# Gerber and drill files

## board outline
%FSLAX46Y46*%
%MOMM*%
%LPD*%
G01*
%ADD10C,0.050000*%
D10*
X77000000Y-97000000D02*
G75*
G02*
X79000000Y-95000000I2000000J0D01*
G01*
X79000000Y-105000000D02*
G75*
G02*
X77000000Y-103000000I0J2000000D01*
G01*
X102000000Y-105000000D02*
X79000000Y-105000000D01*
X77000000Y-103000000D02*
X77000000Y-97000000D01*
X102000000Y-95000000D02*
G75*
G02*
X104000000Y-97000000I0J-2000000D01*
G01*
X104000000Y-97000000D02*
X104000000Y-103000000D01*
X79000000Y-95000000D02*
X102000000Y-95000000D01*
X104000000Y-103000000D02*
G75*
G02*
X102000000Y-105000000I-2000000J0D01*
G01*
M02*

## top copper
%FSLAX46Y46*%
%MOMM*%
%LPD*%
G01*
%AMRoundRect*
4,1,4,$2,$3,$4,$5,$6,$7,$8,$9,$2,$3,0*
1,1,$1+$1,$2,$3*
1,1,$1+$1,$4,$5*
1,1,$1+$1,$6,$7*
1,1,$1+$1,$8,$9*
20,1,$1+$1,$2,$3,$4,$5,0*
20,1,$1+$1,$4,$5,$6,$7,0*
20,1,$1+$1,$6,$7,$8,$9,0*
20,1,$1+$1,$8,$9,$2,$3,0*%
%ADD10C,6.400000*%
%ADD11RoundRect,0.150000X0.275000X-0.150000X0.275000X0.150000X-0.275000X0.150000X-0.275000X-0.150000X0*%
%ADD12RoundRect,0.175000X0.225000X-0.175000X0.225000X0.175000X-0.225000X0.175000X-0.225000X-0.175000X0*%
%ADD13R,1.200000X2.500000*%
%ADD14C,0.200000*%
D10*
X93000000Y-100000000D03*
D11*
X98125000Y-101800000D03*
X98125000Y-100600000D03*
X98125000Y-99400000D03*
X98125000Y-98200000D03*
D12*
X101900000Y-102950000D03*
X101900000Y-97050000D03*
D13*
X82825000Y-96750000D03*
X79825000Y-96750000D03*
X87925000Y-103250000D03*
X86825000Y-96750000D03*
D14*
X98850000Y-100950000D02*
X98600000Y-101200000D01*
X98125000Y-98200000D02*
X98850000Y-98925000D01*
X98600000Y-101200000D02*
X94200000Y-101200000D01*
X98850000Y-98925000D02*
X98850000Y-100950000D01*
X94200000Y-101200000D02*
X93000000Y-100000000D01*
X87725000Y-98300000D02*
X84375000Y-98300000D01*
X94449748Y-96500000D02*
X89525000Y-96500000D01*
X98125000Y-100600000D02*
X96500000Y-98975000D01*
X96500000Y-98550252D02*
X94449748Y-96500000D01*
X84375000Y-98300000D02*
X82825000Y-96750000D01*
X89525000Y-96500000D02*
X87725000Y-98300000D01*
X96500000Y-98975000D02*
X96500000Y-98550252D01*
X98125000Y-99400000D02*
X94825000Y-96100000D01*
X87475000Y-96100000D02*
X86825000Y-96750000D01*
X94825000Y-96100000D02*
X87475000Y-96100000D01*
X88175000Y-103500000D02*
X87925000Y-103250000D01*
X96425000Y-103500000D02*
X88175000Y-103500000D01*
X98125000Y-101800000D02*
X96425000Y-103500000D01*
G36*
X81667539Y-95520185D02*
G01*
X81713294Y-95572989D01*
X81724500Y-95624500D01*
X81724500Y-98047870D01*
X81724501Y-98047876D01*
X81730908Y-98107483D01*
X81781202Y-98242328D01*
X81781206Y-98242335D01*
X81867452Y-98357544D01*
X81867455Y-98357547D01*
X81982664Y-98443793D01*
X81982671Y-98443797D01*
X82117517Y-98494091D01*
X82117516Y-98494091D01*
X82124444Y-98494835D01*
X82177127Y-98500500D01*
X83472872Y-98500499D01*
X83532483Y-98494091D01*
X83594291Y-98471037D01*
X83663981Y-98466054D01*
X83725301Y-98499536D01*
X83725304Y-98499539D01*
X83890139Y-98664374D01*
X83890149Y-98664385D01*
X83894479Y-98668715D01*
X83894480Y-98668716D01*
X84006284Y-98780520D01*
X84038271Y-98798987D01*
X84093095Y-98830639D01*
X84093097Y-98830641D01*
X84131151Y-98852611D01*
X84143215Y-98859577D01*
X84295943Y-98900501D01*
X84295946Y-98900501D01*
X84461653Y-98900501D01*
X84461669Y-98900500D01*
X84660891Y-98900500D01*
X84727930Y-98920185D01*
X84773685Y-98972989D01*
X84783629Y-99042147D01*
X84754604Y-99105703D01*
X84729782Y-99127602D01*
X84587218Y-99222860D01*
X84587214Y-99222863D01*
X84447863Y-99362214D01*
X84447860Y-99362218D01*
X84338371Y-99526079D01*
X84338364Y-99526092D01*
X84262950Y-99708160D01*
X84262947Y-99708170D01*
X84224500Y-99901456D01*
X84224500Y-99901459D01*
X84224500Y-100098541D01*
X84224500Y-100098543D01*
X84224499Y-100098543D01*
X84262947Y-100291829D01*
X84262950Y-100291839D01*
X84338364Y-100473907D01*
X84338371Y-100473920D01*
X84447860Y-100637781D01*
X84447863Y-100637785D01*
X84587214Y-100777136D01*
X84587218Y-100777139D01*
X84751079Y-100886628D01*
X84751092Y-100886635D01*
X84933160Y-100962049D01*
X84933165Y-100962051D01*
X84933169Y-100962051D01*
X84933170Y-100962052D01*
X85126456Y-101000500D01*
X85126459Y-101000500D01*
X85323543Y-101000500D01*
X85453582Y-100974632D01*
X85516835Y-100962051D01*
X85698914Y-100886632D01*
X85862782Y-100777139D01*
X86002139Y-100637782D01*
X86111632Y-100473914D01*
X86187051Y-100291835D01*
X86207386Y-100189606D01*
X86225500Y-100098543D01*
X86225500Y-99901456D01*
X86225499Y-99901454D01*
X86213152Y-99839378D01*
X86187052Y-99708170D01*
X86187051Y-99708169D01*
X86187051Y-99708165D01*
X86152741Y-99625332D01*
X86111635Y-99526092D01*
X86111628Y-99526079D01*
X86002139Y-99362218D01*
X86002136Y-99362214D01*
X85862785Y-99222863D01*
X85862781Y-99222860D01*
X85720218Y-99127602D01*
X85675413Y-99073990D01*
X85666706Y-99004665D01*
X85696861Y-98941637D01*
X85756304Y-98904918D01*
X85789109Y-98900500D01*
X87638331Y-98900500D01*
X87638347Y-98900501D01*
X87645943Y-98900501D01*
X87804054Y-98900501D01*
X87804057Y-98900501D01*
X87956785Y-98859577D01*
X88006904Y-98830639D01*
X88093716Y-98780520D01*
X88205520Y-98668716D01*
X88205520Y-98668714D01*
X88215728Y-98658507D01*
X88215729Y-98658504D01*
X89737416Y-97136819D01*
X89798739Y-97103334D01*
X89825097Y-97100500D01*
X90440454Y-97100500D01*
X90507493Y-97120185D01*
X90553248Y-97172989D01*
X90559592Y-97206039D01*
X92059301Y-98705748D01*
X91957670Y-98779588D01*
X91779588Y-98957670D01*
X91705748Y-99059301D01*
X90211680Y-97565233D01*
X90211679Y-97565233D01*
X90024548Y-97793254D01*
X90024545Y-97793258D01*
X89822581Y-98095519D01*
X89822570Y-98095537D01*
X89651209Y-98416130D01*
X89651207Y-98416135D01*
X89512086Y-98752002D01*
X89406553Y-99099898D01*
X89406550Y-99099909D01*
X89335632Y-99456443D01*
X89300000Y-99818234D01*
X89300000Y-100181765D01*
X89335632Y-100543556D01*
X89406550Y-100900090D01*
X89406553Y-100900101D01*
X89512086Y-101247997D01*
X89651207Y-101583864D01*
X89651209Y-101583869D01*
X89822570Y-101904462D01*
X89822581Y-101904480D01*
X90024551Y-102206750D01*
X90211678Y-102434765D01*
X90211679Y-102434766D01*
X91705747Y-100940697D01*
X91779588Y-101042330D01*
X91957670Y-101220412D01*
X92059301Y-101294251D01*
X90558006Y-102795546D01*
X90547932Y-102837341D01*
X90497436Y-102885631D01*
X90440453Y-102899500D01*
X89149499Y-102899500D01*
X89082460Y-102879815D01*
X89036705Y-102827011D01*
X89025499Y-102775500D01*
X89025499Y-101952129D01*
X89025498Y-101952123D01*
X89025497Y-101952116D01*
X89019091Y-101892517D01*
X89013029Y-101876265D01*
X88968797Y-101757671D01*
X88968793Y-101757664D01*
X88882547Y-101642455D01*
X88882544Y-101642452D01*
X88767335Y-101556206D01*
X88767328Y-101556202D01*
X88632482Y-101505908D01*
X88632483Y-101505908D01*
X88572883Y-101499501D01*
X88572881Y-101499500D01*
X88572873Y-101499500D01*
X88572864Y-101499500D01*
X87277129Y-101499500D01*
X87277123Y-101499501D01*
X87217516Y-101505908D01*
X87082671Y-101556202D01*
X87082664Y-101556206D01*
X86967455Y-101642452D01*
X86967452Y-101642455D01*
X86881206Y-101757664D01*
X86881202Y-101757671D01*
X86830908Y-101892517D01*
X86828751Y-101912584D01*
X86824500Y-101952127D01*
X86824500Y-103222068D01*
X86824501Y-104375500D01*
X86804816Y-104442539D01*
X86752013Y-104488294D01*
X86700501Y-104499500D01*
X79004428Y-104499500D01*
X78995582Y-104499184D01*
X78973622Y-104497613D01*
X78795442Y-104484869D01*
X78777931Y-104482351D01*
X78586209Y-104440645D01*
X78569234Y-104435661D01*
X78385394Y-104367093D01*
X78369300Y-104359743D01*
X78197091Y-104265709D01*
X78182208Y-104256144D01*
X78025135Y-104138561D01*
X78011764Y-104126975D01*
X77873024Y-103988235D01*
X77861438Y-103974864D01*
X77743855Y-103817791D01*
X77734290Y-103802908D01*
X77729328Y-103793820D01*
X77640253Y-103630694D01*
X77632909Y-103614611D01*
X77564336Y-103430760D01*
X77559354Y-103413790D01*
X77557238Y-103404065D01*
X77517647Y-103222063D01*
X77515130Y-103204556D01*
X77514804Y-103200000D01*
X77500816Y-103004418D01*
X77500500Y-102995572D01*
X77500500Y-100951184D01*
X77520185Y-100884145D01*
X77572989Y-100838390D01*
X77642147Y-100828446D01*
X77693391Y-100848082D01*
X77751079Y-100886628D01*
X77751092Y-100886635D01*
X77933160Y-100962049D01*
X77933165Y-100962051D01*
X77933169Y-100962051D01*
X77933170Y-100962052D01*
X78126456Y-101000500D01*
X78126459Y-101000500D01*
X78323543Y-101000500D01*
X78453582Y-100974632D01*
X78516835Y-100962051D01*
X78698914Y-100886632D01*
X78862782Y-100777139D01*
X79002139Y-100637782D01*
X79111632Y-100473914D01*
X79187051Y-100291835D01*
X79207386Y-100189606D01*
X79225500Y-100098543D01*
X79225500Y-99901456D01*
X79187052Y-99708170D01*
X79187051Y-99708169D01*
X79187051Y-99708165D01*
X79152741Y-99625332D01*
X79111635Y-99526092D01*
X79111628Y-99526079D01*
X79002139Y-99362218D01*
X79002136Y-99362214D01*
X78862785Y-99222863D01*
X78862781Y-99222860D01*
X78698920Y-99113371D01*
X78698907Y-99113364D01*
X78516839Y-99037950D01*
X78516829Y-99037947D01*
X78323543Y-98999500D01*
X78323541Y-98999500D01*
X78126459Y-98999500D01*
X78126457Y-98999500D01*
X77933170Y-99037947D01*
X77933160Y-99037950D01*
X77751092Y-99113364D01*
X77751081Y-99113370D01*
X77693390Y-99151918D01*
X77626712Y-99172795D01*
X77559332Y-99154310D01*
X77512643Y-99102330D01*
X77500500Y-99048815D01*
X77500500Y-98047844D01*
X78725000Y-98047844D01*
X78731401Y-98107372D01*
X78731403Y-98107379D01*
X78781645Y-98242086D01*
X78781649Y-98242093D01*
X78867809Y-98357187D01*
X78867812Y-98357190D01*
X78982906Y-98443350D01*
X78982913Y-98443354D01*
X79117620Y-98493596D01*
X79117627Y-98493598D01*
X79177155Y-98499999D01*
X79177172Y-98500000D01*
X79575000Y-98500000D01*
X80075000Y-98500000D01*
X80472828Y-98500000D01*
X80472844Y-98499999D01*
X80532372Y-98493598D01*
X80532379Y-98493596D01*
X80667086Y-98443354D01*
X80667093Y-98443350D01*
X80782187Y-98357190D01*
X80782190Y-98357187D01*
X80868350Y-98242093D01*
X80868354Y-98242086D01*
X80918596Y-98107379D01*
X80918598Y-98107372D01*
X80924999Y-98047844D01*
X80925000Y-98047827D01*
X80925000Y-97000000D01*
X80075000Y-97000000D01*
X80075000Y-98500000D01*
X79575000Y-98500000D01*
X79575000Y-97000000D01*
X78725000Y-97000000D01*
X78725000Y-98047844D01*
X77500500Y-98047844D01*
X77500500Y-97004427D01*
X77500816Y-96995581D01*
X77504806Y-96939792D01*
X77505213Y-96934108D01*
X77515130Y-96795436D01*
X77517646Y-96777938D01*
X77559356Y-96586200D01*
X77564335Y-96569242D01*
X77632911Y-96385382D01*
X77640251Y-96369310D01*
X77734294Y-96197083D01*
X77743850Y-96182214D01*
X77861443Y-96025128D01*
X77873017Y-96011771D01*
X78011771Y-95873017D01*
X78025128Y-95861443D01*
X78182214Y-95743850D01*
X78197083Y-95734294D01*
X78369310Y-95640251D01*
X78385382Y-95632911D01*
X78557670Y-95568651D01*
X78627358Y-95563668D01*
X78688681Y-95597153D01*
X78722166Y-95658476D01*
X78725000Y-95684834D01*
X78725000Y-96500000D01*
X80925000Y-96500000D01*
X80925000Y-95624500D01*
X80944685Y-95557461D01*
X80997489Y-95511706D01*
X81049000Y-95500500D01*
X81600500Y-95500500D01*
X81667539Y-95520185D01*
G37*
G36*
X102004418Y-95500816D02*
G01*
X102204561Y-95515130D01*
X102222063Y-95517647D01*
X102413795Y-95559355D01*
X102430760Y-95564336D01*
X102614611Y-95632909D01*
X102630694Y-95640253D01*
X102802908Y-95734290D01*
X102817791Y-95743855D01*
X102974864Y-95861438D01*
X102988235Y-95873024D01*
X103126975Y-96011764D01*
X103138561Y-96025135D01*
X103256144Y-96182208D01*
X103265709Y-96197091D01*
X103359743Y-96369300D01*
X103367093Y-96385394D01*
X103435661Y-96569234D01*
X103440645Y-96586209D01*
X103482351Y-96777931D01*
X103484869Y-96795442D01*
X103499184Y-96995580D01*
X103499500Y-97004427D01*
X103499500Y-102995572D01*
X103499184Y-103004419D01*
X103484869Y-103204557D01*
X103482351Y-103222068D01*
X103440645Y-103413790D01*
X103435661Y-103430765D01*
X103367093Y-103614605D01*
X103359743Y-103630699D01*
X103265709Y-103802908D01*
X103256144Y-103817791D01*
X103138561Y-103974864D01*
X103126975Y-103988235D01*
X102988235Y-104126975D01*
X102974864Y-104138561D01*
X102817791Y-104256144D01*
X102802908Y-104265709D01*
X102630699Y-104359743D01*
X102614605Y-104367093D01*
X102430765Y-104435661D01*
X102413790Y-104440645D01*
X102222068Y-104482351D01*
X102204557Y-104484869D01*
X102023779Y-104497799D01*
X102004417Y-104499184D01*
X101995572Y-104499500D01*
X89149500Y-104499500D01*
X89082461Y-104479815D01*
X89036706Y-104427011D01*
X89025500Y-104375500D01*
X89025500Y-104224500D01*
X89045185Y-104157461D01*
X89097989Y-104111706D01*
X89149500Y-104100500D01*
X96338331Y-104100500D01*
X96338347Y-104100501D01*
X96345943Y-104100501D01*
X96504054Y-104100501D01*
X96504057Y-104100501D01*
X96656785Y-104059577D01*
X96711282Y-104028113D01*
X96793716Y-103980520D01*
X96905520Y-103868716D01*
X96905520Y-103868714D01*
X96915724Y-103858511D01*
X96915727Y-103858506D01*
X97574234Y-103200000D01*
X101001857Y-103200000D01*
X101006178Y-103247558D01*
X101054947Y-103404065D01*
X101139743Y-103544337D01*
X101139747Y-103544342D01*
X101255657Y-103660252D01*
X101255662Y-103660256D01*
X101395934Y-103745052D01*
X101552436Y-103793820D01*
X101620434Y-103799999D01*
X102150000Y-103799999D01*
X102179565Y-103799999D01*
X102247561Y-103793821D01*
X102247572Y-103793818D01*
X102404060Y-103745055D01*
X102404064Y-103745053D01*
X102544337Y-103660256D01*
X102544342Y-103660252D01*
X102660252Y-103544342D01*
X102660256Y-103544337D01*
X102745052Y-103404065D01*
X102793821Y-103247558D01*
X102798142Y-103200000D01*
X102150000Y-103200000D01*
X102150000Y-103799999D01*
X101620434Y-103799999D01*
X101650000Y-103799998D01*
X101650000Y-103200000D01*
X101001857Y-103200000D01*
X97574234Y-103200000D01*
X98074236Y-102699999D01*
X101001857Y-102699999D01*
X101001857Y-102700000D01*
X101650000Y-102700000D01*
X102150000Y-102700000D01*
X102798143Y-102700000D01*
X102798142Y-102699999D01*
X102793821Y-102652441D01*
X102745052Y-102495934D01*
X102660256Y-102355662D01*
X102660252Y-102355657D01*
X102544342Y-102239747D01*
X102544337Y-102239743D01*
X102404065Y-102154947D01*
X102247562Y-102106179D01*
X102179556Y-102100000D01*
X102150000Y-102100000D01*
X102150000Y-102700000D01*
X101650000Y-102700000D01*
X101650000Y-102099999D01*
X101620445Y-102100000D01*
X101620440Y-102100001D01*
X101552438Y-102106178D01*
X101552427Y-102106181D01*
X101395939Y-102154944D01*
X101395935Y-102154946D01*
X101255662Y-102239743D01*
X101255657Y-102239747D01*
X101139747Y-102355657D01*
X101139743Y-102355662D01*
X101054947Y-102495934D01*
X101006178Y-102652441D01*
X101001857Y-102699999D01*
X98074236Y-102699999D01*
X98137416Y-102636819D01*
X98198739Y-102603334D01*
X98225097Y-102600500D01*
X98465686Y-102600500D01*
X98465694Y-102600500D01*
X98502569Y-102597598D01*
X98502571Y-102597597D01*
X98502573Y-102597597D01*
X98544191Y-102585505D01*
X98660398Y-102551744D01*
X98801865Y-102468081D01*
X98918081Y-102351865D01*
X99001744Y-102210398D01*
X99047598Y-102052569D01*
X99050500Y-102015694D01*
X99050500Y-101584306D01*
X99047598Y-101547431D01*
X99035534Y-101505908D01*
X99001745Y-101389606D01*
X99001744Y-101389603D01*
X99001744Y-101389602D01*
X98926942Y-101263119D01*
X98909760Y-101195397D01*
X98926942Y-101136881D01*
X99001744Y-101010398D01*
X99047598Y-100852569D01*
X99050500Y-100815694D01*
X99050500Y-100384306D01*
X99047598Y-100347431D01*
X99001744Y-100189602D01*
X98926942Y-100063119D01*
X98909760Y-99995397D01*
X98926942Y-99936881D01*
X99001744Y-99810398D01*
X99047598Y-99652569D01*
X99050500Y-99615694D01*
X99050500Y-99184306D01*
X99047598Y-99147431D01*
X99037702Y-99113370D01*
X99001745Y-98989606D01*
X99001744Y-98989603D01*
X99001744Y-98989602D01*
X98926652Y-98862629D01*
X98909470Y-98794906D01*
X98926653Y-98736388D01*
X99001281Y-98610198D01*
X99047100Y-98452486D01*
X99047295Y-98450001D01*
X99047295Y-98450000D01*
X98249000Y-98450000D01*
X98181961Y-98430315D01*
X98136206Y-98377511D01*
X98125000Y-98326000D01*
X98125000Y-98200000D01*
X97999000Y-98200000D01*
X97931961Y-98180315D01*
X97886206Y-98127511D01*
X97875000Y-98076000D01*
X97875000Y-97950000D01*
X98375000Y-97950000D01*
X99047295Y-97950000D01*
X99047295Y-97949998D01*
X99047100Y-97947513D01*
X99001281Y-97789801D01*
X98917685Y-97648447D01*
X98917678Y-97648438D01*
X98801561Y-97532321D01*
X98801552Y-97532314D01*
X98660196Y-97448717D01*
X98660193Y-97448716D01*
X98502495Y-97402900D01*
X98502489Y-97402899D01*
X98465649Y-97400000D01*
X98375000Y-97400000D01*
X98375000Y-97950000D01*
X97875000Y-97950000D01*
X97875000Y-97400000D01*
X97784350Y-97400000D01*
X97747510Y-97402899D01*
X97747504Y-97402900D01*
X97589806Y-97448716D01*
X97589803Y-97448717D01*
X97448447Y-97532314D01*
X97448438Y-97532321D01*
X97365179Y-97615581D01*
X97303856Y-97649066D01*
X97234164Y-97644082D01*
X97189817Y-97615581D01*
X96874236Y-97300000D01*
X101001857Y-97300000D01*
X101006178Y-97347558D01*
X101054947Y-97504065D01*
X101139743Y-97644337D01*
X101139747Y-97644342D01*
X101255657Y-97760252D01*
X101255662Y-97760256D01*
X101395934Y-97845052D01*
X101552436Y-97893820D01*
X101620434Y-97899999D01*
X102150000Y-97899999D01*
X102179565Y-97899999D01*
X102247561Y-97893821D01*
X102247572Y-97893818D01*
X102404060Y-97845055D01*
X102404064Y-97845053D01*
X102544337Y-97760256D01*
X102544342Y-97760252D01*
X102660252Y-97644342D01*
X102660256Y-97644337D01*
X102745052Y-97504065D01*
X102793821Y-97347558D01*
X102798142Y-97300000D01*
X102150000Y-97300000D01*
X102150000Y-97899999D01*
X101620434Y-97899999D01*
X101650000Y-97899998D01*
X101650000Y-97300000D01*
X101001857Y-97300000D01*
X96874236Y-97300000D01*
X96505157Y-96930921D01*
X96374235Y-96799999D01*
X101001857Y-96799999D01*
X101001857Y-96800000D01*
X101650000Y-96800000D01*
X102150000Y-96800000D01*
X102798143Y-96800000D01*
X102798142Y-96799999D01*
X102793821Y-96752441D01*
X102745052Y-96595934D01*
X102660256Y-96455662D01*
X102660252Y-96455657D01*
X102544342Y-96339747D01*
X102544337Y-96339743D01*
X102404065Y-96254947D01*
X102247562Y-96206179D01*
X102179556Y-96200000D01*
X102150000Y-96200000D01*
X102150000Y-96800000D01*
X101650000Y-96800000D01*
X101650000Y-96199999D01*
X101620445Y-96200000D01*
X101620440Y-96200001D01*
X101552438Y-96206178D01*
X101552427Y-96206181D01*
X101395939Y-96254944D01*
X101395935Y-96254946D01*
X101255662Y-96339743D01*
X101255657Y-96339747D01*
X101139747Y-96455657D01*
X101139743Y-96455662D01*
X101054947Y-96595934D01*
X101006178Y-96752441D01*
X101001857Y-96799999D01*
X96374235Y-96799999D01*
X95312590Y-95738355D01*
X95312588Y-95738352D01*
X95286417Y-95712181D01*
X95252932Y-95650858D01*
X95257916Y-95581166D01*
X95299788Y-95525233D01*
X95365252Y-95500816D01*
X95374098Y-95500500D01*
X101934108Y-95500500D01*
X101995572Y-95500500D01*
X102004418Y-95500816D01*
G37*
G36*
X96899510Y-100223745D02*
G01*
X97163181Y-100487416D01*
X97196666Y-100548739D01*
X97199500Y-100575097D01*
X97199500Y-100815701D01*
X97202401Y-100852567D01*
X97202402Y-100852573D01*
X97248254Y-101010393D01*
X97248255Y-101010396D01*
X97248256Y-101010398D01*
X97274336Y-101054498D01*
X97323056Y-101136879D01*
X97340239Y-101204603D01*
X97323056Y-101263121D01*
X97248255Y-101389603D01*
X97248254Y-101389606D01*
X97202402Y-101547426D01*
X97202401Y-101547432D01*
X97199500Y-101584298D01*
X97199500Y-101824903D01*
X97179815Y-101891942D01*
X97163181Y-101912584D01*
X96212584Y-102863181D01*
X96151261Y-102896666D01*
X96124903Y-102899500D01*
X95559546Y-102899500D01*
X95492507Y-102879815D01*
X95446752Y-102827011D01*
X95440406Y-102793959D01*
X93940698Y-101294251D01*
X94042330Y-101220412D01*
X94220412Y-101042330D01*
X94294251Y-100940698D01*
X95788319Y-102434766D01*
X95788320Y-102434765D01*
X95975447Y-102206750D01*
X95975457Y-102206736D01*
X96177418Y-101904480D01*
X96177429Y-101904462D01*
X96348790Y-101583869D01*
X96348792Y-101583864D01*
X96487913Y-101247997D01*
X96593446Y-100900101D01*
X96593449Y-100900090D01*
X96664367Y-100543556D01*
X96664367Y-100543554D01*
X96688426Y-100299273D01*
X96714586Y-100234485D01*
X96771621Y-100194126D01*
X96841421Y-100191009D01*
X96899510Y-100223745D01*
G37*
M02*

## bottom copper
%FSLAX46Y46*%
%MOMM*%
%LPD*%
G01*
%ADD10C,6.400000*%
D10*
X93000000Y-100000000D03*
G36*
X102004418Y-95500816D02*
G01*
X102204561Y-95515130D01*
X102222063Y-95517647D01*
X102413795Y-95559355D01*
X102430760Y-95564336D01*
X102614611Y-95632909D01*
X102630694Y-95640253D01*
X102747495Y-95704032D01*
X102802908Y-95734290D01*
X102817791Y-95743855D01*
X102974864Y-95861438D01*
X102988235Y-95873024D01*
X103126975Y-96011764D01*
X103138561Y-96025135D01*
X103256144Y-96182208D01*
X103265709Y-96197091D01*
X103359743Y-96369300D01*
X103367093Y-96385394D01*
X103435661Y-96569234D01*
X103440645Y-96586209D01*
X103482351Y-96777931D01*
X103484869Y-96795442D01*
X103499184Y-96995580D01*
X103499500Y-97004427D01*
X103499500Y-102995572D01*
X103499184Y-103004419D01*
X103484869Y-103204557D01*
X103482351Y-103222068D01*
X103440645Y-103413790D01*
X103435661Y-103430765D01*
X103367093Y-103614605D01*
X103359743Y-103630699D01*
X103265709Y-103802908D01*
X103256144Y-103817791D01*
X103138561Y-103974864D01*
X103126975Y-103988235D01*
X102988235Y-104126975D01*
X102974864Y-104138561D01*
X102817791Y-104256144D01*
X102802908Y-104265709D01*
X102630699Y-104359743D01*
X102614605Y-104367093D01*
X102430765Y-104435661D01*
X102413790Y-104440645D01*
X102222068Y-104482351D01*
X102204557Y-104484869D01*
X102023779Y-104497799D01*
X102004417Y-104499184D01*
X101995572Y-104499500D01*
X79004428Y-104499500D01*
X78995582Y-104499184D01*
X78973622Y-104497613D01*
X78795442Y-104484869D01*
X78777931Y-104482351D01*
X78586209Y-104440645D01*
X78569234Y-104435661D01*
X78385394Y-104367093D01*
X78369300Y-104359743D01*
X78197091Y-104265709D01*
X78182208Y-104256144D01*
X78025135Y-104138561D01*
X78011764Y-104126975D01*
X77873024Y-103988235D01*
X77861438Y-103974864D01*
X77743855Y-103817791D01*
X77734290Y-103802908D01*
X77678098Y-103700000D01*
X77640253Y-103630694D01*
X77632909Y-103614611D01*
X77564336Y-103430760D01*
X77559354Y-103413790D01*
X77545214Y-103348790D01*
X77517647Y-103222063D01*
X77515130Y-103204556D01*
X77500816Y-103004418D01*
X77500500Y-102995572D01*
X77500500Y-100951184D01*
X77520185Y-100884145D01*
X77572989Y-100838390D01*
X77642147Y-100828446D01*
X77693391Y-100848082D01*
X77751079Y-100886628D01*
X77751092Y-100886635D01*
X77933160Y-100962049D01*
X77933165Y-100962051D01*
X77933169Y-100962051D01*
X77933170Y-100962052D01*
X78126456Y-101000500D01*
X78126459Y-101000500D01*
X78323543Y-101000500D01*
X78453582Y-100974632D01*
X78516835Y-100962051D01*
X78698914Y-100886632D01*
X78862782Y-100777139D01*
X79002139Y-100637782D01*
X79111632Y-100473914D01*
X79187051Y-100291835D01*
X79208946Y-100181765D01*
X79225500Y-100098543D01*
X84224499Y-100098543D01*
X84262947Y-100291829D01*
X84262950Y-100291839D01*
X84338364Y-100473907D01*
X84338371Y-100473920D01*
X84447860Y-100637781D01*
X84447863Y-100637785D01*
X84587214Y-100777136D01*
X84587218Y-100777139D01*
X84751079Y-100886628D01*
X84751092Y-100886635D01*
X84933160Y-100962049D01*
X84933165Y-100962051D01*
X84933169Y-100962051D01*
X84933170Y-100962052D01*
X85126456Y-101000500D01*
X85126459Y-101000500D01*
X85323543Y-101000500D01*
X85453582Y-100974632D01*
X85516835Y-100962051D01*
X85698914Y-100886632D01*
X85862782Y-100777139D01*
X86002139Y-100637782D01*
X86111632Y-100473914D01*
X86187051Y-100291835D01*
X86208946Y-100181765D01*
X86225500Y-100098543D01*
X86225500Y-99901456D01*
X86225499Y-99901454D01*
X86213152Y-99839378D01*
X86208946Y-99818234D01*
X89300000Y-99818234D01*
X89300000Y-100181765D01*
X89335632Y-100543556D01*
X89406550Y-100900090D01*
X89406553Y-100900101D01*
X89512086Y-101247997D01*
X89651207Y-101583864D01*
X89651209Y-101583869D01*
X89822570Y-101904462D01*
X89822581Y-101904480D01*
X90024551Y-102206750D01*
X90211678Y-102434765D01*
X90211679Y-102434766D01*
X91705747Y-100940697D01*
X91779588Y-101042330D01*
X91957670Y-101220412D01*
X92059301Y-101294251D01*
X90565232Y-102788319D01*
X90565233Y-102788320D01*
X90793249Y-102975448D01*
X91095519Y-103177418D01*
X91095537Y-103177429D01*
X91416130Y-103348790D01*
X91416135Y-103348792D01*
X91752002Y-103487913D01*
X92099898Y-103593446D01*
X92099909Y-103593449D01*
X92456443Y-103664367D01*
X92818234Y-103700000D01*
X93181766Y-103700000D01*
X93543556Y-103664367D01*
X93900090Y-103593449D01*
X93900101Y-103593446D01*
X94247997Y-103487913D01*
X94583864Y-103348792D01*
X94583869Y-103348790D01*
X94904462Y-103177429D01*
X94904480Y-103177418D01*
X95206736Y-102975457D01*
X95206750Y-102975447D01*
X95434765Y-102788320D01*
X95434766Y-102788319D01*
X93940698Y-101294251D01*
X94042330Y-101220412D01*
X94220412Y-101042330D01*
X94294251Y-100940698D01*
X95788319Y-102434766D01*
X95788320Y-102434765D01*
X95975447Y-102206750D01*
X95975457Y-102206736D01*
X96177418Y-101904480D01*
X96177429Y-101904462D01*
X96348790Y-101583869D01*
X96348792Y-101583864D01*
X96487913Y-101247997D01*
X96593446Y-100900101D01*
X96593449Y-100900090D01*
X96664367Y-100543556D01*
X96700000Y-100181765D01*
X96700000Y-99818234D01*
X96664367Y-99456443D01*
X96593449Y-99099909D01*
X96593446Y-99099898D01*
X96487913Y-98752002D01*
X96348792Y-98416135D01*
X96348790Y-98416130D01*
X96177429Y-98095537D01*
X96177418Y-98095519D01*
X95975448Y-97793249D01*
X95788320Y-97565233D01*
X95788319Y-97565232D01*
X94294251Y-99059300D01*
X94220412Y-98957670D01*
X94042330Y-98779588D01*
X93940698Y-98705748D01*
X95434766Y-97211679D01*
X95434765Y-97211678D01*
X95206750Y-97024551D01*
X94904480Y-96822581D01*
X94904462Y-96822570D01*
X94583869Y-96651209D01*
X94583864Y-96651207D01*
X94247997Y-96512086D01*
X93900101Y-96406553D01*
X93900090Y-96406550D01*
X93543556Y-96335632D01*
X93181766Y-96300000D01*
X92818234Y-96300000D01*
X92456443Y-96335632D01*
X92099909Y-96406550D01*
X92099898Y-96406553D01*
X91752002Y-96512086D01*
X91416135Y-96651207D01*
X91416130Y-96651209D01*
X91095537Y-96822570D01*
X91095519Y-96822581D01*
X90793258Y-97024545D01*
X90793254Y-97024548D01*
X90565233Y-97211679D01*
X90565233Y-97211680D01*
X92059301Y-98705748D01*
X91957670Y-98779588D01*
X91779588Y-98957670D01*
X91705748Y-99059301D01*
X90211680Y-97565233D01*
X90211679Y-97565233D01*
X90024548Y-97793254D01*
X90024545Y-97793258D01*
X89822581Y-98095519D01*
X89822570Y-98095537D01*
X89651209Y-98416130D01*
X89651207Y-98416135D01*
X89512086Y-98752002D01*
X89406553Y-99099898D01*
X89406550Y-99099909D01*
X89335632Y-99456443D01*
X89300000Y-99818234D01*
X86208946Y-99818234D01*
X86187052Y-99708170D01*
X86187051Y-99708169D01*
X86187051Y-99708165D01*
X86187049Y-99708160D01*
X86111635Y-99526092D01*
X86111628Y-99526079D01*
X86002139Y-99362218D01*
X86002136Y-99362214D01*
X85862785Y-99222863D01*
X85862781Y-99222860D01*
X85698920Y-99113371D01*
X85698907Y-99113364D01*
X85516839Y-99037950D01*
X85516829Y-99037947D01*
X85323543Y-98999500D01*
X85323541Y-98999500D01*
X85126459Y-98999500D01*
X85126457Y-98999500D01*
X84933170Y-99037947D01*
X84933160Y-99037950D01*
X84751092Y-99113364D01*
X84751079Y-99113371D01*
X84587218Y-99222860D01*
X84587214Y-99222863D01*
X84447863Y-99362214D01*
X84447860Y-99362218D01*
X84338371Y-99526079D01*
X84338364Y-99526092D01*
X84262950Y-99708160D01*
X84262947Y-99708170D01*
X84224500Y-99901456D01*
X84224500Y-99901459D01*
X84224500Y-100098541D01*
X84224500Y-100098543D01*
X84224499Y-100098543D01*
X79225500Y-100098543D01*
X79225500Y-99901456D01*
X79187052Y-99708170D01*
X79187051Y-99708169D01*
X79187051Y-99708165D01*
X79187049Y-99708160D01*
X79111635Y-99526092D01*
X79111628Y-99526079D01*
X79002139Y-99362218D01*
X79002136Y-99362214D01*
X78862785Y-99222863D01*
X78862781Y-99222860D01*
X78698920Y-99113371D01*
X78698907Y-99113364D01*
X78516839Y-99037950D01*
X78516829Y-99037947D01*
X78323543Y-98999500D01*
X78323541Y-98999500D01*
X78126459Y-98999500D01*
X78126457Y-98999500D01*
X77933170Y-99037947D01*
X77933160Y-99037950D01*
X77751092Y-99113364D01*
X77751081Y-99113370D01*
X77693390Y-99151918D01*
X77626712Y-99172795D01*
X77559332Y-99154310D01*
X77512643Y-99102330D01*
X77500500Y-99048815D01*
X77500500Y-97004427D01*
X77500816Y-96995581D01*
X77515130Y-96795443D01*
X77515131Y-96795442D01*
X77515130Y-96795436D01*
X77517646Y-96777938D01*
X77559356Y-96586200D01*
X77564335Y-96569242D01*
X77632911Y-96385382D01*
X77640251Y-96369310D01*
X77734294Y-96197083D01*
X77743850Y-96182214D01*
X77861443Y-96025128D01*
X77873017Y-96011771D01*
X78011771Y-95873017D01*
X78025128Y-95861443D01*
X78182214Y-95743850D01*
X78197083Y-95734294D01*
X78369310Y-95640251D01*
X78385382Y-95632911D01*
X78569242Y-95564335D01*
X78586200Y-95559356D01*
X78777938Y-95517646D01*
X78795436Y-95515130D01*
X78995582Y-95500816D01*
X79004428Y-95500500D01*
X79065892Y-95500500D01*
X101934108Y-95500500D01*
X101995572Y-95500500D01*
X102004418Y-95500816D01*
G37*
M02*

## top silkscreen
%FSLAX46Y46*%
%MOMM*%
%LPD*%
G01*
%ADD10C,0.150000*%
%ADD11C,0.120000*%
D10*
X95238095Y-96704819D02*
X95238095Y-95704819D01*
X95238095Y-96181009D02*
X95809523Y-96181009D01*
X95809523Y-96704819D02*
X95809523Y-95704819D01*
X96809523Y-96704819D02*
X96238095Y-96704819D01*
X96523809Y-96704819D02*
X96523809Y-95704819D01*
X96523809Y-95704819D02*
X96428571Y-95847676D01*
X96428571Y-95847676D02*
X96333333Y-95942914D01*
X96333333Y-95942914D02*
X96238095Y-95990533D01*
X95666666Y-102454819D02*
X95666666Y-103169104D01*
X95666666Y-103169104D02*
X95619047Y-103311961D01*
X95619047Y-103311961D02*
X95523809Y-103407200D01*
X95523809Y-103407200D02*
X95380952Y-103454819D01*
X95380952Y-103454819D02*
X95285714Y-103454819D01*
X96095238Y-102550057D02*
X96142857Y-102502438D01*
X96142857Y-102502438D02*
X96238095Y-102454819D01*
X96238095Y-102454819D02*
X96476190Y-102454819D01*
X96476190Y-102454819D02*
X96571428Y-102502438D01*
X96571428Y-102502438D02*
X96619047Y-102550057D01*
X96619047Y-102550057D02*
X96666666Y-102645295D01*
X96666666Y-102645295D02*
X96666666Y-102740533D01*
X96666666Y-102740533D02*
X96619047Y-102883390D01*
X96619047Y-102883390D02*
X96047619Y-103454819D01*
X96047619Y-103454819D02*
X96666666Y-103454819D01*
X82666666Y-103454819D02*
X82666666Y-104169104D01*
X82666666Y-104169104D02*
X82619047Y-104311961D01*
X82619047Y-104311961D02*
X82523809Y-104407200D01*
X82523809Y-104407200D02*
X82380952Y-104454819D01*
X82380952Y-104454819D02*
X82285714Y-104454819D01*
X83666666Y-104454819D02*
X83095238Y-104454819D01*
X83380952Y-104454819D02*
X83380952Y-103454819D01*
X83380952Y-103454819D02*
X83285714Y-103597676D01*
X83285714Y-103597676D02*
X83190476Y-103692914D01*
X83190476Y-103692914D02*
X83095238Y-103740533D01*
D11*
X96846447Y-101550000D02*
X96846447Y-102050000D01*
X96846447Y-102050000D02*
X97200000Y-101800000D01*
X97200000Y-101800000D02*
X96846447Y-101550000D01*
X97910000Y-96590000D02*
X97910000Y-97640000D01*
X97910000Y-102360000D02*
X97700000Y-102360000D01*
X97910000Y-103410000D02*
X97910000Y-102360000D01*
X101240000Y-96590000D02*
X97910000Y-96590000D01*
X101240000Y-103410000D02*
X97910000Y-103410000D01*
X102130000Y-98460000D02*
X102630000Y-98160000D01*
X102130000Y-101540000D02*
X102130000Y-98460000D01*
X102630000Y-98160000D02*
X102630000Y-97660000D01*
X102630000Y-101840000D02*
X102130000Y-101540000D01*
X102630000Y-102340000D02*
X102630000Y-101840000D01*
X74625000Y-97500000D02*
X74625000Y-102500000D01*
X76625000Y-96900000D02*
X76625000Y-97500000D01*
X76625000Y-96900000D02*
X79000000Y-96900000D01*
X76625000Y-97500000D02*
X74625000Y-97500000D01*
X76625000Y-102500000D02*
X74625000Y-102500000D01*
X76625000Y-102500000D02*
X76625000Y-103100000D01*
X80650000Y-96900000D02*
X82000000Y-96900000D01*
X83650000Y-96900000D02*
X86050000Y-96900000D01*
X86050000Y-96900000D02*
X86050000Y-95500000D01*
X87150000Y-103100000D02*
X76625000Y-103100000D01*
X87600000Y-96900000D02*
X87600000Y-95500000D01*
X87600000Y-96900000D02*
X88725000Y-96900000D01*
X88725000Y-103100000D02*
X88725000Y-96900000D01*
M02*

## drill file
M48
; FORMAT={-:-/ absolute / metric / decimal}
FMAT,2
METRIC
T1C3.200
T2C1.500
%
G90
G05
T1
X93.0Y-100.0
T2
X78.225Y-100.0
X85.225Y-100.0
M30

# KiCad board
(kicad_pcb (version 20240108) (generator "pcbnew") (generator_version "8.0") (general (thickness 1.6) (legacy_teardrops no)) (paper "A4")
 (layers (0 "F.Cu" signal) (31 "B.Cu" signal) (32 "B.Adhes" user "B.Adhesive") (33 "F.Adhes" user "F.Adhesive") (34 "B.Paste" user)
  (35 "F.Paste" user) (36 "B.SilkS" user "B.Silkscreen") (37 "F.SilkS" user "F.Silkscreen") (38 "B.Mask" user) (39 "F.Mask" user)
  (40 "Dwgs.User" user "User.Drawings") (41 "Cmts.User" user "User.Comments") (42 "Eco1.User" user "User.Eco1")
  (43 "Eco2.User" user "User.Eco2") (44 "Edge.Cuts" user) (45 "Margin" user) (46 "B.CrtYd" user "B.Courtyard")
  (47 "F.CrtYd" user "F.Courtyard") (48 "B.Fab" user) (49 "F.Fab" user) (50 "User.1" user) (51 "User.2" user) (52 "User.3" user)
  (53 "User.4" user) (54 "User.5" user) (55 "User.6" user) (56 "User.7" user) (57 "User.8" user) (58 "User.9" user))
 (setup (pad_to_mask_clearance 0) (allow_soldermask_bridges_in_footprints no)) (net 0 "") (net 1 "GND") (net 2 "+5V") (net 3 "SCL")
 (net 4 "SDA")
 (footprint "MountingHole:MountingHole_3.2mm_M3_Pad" (layer "F.Cu") (at 93 100)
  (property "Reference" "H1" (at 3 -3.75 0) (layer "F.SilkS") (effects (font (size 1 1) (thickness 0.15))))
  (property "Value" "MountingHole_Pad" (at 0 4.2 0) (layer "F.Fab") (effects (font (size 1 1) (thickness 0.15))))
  (pad "1" thru_hole circle (at 0 0) (size 6.4 6.4) (drill 3.2) (layers "*.Cu" "*.Mask") (remove_unused_layers no) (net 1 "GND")))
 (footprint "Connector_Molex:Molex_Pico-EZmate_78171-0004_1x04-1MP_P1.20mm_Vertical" (layer "F.Cu") (at 100 100 90)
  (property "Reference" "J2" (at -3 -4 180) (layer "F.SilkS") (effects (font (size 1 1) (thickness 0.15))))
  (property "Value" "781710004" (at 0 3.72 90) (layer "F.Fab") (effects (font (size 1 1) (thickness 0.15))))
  (fp_line (start -1.55 -3.153553) (end -2.05 -3.153553) (stroke (width 0.12) (type solid)) (layer "F.SilkS"))
  (fp_line (start -2.05 -3.153553) (end -1.8 -2.8) (stroke (width 0.12) (type solid)) (layer "F.SilkS"))
  (fp_line (start -1.8 -2.8) (end -1.55 -3.153553) (stroke (width 0.12) (type solid)) (layer "F.SilkS"))
  (fp_line (start 3.41 -2.09) (end 2.36 -2.09) (stroke (width 0.12) (type solid)) (layer "F.SilkS"))
  (fp_line (start -2.36 -2.09) (end -2.36 -2.3) (stroke (width 0.12) (type solid)) (layer "F.SilkS"))
  (fp_line (start -3.41 -2.09) (end -2.36 -2.09) (stroke (width 0.12) (type solid)) (layer "F.SilkS"))
  (fp_line (start 3.41 1.24) (end 3.41 -2.09) (stroke (width 0.12) (type solid)) (layer "F.SilkS"))
  (fp_line (start -3.41 1.24) (end -3.41 -2.09) (stroke (width 0.12) (type solid)) (layer "F.SilkS"))
  (fp_line (start 1.54 2.13) (end 1.84 2.63) (stroke (width 0.12) (type solid)) (layer "F.SilkS"))
  (fp_line (start -1.54 2.13) (end 1.54 2.13) (stroke (width 0.12) (type solid)) (layer "F.SilkS"))
  (fp_line (start 1.84 2.63) (end 2.34 2.63) (stroke (width 0.12) (type solid)) (layer "F.SilkS"))
  (fp_line (start -1.84 2.63) (end -1.54 2.13) (stroke (width 0.12) (type solid)) (layer "F.SilkS"))
  (fp_line (start -2.34 2.63) (end -1.84 2.63) (stroke (width 0.12) (type solid)) (layer "F.SilkS"))
  (pad "1" smd roundrect (at -1.8 -1.875 90) (size 0.6 0.85) (layers "F.Cu" "F.Paste" "F.Mask") (roundrect_rratio 0.25) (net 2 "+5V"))
  (pad "2" smd roundrect (at -0.6 -1.875 90) (size 0.6 0.85) (layers "F.Cu" "F.Paste" "F.Mask") (roundrect_rratio 0.25) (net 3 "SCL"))
  (pad "3" smd roundrect (at 0.6 -1.875 90) (size 0.6 0.85) (layers "F.Cu" "F.Paste" "F.Mask") (roundrect_rratio 0.25) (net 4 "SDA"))
  (pad "4" smd roundrect (at 1.8 -1.875 90) (size 0.6 0.85) (layers "F.Cu" "F.Paste" "F.Mask") (roundrect_rratio 0.25) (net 1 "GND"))
  (pad "MP" smd roundrect (at -2.95 1.9 90) (size 0.7 0.8) (layers "F.Cu" "F.Paste" "F.Mask") (roundrect_rratio 0.25) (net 1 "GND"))
  (pad "MP" smd roundrect (at 2.95 1.9 90) (size 0.7 0.8) (layers "F.Cu" "F.Paste" "F.Mask") (roundrect_rratio 0.25) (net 1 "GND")))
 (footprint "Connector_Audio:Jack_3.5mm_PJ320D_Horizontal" (layer "F.Cu") (at 83 100)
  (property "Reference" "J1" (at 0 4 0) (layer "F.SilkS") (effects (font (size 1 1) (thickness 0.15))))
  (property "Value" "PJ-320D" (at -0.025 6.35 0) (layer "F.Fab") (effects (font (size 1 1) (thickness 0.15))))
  (fp_line (start -8.375 -2.5) (end -8.375 2.5) (stroke (width 0.12) (type solid)) (layer "F.SilkS"))
  (fp_line (start -6.375 -3.1) (end -6.375 -2.5) (stroke (width 0.12) (type solid)) (layer "F.SilkS"))
  (fp_line (start -6.375 -3.1) (end -4 -3.1) (stroke (width 0.12) (type solid)) (layer "F.SilkS"))
  (fp_line (start -6.375 -2.5) (end -8.375 -2.5) (stroke (width 0.12) (type solid)) (layer "F.SilkS"))
  (fp_line (start -6.375 2.5) (end -8.375 2.5) (stroke (width 0.12) (type solid)) (layer "F.SilkS"))
  (fp_line (start -6.375 2.5) (end -6.375 3.1) (stroke (width 0.12) (type solid)) (layer "F.SilkS"))
  (fp_line (start -2.35 -3.1) (end -1 -3.1) (stroke (width 0.12) (type solid)) (layer "F.SilkS"))
  (fp_line (start 0.65 -3.1) (end 3.05 -3.1) (stroke (width 0.12) (type solid)) (layer "F.SilkS"))
  (fp_line (start 3.05 -3.1) (end 3.05 -4.5) (stroke (width 0.12) (type solid)) (layer "F.SilkS"))
  (fp_line (start 4.15 3.1) (end -6.375 3.1) (stroke (width 0.12) (type solid)) (layer "F.SilkS"))
  (fp_line (start 4.6 -3.1) (end 4.6 -4.5) (stroke (width 0.12) (type solid)) (layer "F.SilkS"))
  (fp_line (start 4.6 -3.1) (end 5.725 -3.1) (stroke (width 0.12) (type solid)) (layer "F.SilkS"))
  (fp_line (start 5.725 3.1) (end 5.725 -3.1) (stroke (width 0.12) (type solid)) (layer "F.SilkS"))
  (pad "" np_thru_hole circle (at -4.775 0) (size 1.5 1.5) (drill 1.5) (layers "*.Cu" "*.Mask"))
  (pad "" np_thru_hole circle (at 2.225 0) (size 1.5 1.5) (drill 1.5) (layers "*.Cu" "*.Mask"))
  (pad "R1" smd rect (at -0.175 -3.25) (size 1.2 2.5) (layers "F.Cu" "F.Paste" "F.Mask") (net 3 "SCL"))
  (pad "R2" smd rect (at -3.175 -3.25) (size 1.2 2.5) (layers "F.Cu" "F.Paste" "F.Mask") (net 1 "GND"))
  (pad "S" smd rect (at 4.925 3.25) (size 1.2 2.5) (layers "F.Cu" "F.Paste" "F.Mask") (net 2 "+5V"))
  (pad "T" smd rect (at 3.825 -3.25) (size 1.2 2.5) (layers "F.Cu" "F.Paste" "F.Mask") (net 4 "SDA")))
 (gr_arc (start 77 97) (mid 77.585786 95.585786) (end 79 95) (stroke (width 0.05) (type default)) (layer "Edge.Cuts"))
 (gr_arc (start 79 105) (mid 77.585786 104.414214) (end 77 103) (stroke (width 0.05) (type default)) (layer "Edge.Cuts"))
 (gr_line (start 102 105) (end 79 105) (stroke (width 0.05) (type default)) (layer "Edge.Cuts"))
 (gr_line (start 77 103) (end 77 97) (stroke (width 0.05) (type default)) (layer "Edge.Cuts"))
 (gr_arc (start 102 95) (mid 103.414214 95.585786) (end 104 97) (stroke (width 0.05) (type default)) (layer "Edge.Cuts"))
 (gr_line (start 104 97) (end 104 103) (stroke (width 0.05) (type default)) (layer "Edge.Cuts"))
 (gr_line (start 79 95) (end 102 95) (stroke (width 0.05) (type default)) (layer "Edge.Cuts"))
 (gr_arc (start 104 103) (mid 103.414214 104.414214) (end 102 105) (stroke (width 0.05) (type default)) (layer "Edge.Cuts"))
 (segment (start 98.85 100.95) (end 98.6 101.2) (width 0.2) (layer "F.Cu") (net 1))
 (segment (start 98.125 98.2) (end 98.85 98.925) (width 0.2) (layer "F.Cu") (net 1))
 (segment (start 98.6 101.2) (end 94.2 101.2) (width 0.2) (layer "F.Cu") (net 1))
 (segment (start 98.85 98.925) (end 98.85 100.95) (width 0.2) (layer "F.Cu") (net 1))
 (segment (start 94.2 101.2) (end 93 100) (width 0.2) (layer "F.Cu") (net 1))
 (segment (start 87.725 98.3) (end 84.375 98.3) (width 0.2) (layer "F.Cu") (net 3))
 (segment (start 94.449748 96.5) (end 89.525 96.5) (width 0.2) (layer "F.Cu") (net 3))
 (segment (start 98.125 100.6) (end 96.5 98.975) (width 0.2) (layer "F.Cu") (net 3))
 (segment (start 96.5 98.550252) (end 94.449748 96.5) (width 0.2) (layer "F.Cu") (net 3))
 (segment (start 84.375 98.3) (end 82.825 96.75) (width 0.2) (layer "F.Cu") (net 3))
 (segment (start 89.525 96.5) (end 87.725 98.3) (width 0.2) (layer "F.Cu") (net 3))
 (segment (start 96.5 98.975) (end 96.5 98.550252) (width 0.2) (layer "F.Cu") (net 3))
 (segment (start 98.125 99.4) (end 94.825 96.1) (width 0.2) (layer "F.Cu") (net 4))
 (segment (start 87.475 96.1) (end 86.825 96.75) (width 0.2) (layer "F.Cu") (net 4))
 (segment (start 94.825 96.1) (end 87.475 96.1) (width 0.2) (layer "F.Cu") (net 4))
 (segment (start 88.175 103.5) (end 87.925 103.25) (width 0.2) (layer "F.Cu") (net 2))
 (segment (start 96.425 103.5) (end 88.175 103.5) (width 0.2) (layer "F.Cu") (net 2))
 (segment (start 98.125 101.8) (end 96.425 103.5) (width 0.2) (layer "F.Cu") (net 2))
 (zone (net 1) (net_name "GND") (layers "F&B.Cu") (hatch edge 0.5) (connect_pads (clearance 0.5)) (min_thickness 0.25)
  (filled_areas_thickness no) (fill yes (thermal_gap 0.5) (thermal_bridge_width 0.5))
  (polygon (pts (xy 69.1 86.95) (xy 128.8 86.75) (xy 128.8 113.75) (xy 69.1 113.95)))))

